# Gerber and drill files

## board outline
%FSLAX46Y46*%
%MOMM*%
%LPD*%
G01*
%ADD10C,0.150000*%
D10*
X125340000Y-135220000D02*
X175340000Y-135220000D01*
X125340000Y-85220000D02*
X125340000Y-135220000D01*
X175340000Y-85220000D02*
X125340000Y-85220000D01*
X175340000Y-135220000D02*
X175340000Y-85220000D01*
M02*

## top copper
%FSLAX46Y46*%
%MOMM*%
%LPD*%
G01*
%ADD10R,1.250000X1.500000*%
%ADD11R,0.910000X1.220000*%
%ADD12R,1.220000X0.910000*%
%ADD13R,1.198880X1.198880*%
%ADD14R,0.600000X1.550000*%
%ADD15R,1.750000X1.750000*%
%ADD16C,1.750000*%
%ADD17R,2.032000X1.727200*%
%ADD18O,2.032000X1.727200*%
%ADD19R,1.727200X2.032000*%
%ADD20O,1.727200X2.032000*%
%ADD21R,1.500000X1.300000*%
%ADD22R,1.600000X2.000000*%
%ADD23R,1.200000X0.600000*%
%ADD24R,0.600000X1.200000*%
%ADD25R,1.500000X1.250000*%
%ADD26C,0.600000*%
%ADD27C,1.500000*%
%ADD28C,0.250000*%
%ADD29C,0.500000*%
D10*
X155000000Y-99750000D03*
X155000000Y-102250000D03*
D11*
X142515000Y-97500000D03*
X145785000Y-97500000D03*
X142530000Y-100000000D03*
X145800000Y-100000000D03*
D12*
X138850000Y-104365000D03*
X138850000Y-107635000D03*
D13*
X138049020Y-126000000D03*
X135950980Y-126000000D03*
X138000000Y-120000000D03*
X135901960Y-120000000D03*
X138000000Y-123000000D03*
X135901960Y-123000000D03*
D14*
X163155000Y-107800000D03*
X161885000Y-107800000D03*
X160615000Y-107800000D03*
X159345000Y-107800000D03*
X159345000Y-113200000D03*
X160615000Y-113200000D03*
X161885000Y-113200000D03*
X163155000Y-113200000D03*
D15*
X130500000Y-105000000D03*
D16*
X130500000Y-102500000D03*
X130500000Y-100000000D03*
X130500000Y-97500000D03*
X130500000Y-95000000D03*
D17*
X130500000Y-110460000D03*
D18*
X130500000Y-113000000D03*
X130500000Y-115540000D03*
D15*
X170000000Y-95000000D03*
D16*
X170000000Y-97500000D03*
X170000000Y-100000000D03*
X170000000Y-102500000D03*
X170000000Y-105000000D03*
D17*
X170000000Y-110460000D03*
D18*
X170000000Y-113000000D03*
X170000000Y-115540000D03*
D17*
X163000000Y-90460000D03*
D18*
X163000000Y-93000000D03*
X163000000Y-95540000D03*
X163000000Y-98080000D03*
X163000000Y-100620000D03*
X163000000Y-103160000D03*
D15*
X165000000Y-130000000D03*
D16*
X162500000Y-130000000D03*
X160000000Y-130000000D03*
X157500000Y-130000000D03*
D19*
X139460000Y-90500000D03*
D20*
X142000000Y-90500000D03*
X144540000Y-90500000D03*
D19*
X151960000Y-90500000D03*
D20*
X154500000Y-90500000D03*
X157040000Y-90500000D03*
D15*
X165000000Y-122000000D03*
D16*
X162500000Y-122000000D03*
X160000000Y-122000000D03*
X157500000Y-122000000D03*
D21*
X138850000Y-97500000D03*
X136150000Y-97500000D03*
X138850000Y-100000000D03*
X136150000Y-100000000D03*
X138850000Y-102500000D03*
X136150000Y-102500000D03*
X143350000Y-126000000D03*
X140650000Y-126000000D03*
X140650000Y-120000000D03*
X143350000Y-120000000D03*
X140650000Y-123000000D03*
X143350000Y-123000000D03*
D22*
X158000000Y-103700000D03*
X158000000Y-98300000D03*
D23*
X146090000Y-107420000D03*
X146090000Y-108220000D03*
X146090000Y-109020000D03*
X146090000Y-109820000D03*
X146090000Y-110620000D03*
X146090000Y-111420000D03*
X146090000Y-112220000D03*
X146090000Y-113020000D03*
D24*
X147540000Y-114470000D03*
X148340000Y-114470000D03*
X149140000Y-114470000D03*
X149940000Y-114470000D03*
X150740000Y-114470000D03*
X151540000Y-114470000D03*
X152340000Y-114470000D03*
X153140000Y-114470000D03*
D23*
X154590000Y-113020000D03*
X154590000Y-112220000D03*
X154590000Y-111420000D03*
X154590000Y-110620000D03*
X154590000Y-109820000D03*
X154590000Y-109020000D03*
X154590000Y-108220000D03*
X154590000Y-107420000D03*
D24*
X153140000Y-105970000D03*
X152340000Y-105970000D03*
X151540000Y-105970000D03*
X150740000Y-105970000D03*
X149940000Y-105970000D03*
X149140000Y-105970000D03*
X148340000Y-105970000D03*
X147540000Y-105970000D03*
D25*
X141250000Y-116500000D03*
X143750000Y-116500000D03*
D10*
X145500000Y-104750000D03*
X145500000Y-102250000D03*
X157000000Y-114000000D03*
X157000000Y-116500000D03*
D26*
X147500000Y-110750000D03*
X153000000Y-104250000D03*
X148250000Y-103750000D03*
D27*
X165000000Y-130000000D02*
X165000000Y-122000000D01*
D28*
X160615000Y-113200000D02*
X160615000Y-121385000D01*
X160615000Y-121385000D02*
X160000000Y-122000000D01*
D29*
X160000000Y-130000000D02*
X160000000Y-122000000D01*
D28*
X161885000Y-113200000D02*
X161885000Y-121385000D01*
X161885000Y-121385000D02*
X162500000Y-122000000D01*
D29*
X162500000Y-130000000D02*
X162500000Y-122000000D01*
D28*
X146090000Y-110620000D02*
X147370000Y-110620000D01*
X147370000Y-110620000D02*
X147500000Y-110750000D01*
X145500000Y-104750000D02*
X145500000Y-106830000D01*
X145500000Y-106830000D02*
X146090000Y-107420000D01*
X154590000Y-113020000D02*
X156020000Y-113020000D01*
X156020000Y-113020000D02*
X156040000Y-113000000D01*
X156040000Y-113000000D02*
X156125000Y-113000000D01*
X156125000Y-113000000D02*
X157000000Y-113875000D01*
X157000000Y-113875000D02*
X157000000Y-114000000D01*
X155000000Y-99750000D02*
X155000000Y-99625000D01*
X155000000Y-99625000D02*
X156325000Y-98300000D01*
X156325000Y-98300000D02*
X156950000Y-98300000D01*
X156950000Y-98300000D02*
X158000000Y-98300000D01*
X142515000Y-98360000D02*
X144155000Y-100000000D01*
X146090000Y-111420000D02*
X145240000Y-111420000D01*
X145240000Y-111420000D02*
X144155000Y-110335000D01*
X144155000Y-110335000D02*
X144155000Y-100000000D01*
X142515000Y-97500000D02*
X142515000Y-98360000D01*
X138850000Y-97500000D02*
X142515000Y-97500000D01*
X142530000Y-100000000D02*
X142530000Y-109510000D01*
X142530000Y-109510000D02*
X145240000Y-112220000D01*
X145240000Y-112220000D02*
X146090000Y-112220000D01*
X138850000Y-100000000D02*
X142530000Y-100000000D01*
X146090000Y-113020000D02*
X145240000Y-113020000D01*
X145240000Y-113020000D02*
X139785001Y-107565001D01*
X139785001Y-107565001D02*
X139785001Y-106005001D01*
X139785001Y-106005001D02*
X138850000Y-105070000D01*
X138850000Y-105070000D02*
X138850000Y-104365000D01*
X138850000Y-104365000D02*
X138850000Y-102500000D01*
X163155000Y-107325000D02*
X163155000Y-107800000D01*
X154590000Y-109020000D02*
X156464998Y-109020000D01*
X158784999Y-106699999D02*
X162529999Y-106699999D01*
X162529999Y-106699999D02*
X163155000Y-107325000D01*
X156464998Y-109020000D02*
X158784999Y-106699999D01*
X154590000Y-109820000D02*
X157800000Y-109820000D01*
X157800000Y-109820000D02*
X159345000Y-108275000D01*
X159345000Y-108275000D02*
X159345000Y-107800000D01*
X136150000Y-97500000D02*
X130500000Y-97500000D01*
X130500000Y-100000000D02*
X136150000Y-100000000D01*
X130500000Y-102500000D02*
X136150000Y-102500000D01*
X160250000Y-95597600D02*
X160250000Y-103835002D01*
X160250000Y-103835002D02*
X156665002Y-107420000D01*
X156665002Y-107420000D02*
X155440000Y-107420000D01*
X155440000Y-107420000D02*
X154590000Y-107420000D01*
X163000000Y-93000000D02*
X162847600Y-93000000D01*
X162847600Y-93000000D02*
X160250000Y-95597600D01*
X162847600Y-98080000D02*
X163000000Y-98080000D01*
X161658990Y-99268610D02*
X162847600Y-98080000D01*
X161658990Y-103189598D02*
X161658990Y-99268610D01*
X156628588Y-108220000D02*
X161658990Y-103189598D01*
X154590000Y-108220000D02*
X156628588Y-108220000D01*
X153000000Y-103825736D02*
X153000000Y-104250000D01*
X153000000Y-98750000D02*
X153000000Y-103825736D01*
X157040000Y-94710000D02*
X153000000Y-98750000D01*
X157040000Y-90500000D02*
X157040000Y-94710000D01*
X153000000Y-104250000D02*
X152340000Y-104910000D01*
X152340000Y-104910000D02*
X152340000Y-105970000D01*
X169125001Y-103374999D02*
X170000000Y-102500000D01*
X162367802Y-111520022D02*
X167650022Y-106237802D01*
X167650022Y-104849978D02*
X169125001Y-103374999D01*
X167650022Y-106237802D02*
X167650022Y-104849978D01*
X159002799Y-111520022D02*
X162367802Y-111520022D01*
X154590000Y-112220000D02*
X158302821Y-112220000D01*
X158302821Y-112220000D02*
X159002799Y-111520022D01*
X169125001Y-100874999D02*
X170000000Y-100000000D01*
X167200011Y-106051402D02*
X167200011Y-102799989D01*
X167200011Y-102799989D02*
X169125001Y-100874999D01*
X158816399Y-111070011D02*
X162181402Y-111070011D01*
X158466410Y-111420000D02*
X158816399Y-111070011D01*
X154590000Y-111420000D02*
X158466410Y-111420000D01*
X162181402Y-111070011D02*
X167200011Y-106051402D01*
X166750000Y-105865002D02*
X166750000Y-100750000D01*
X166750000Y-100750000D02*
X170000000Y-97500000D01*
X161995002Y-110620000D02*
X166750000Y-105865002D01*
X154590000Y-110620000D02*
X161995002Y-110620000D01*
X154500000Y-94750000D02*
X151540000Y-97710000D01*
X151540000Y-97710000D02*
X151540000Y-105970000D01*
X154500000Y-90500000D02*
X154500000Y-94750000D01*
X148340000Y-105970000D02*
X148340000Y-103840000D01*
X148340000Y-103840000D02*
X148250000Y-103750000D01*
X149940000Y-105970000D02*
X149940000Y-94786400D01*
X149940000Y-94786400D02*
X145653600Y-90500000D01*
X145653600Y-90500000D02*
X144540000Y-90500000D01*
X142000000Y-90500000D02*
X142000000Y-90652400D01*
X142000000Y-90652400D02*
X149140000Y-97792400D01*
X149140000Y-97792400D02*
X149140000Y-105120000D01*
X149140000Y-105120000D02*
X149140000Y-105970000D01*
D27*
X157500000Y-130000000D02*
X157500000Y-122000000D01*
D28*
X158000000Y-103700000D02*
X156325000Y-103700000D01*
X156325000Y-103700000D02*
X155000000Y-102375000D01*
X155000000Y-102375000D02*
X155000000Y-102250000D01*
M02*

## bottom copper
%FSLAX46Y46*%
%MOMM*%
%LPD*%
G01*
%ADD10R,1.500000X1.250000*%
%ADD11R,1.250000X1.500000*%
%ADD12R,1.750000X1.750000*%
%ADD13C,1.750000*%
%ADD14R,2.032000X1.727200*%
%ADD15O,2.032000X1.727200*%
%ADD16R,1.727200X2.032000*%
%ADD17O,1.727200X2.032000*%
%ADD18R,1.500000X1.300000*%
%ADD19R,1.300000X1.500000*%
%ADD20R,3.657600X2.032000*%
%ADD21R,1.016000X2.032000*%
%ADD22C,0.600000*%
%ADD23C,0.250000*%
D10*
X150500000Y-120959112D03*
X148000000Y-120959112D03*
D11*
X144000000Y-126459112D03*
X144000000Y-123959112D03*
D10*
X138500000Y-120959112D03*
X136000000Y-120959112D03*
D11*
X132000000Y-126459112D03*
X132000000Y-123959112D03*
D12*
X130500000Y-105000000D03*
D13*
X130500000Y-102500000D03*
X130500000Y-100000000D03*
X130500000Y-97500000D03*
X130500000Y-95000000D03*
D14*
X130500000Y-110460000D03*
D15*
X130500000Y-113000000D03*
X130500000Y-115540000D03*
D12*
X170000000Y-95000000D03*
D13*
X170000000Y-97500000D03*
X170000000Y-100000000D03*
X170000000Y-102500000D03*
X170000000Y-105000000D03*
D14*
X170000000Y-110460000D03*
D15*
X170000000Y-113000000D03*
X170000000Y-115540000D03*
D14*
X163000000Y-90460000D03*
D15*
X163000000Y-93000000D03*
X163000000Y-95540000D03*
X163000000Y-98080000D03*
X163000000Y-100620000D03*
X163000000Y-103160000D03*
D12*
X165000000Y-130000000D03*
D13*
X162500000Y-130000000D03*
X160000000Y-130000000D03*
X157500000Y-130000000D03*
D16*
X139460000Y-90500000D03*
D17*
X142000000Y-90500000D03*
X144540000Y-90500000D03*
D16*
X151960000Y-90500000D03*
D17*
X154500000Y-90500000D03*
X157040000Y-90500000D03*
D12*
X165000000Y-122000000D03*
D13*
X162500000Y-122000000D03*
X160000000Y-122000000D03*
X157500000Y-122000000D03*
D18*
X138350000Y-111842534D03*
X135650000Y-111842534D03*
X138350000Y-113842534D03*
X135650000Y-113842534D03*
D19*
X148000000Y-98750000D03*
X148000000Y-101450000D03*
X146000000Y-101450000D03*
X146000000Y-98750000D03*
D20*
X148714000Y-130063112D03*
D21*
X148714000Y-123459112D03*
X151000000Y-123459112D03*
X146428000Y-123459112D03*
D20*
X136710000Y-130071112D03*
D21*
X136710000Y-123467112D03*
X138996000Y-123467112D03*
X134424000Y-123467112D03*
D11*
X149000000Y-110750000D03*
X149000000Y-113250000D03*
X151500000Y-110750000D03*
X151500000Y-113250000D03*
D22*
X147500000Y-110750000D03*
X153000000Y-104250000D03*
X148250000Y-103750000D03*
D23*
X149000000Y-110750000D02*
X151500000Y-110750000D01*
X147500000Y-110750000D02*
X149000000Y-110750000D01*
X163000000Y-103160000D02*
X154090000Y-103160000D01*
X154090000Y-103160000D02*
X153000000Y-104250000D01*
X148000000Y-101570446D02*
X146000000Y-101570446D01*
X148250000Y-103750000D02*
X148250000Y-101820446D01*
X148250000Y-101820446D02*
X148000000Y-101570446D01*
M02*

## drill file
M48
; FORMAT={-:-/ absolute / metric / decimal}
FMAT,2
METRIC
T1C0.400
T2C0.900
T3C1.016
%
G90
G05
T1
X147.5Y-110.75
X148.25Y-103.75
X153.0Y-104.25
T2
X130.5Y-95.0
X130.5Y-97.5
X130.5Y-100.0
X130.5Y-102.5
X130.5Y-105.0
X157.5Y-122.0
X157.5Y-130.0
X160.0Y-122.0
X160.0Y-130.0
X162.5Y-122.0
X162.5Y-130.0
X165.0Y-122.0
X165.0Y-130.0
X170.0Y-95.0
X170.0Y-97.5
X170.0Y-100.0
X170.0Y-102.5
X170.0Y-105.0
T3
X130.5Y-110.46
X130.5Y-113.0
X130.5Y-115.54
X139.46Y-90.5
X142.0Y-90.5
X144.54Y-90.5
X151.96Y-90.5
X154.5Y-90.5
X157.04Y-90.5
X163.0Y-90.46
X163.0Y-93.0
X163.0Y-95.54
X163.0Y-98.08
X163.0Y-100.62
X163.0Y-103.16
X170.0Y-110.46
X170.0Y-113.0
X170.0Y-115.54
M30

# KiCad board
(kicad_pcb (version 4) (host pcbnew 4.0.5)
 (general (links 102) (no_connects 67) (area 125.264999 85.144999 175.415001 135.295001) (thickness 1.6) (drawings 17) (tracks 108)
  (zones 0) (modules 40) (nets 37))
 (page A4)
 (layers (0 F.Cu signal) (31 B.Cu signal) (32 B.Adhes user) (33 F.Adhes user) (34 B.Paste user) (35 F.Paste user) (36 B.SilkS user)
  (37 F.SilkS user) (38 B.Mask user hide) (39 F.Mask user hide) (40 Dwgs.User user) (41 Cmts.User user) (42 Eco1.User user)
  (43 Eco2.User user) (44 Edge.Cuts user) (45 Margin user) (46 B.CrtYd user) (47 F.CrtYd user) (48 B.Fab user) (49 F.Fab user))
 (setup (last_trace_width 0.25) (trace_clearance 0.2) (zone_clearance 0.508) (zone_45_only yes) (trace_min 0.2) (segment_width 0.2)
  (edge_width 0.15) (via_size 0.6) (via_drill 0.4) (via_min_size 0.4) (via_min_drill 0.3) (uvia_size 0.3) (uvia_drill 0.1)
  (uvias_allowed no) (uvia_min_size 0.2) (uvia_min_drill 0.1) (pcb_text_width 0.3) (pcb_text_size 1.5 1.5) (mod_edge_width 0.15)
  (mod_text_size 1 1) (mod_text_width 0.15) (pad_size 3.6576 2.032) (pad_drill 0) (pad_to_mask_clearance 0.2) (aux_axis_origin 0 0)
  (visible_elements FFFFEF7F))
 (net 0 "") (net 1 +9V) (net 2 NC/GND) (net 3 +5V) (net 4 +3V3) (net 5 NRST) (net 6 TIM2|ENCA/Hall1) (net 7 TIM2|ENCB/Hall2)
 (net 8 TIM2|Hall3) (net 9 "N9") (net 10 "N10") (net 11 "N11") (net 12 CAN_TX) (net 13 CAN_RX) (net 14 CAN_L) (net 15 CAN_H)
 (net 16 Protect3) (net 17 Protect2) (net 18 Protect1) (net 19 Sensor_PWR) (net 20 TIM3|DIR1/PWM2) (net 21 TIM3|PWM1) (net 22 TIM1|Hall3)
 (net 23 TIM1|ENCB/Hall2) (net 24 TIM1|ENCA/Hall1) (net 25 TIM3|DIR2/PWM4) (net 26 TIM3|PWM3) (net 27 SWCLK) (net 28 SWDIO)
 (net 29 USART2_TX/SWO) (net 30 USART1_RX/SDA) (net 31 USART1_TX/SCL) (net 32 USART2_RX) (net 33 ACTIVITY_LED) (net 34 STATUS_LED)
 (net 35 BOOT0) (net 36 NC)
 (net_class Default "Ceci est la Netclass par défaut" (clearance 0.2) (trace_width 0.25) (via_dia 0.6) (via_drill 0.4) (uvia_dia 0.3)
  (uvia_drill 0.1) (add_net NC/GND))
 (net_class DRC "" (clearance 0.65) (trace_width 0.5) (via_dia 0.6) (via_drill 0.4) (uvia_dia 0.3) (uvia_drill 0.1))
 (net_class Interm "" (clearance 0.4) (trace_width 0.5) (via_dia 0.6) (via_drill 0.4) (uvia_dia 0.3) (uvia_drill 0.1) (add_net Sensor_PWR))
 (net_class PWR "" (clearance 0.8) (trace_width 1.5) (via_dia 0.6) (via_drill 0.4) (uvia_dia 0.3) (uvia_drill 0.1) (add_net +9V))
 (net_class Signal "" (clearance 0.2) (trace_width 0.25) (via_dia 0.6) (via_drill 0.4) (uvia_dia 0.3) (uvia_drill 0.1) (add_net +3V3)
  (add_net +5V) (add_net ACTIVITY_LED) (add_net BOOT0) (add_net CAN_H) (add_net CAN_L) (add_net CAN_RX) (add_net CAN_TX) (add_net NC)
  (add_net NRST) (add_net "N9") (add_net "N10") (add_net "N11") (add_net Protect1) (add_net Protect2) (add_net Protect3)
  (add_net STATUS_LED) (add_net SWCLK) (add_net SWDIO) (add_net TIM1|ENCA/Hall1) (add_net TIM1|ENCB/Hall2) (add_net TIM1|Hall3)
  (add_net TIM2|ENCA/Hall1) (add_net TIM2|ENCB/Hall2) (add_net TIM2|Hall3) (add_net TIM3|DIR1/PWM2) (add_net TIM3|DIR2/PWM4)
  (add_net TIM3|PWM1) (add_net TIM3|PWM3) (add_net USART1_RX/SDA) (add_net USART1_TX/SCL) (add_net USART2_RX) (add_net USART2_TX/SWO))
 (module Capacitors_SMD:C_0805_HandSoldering (layer B.Cu) (at 149.25 120.959112 180)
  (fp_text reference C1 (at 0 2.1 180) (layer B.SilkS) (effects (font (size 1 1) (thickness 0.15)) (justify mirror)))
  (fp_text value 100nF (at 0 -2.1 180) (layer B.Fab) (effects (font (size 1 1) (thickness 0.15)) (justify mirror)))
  (pad 1 smd rect (at -1.25 0 180) (size 1.5 1.25) (layers B.Cu B.Paste B.Mask) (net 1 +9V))
  (pad 2 smd rect (at 1.25 0 180) (size 1.5 1.25) (layers B.Cu B.Paste B.Mask) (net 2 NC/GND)))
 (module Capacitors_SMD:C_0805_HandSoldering (layer B.Cu) (at 144 125.209112 90)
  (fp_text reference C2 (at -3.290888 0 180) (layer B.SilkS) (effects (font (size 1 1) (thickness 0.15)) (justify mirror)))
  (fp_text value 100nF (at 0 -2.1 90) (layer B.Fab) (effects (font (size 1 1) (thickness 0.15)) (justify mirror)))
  (pad 1 smd rect (at -1.25 0 90) (size 1.5 1.25) (layers B.Cu B.Paste B.Mask) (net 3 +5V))
  (pad 2 smd rect (at 1.25 0 90) (size 1.5 1.25) (layers B.Cu B.Paste B.Mask) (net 2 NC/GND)))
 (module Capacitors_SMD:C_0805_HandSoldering (layer B.Cu) (at 137.25 120.959112 180)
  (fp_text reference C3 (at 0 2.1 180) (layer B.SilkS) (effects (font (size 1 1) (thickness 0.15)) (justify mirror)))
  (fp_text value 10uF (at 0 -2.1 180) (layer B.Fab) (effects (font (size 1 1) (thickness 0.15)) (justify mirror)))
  (pad 1 smd rect (at -1.25 0 180) (size 1.5 1.25) (layers B.Cu B.Paste B.Mask) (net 3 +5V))
  (pad 2 smd rect (at 1.25 0 180) (size 1.5 1.25) (layers B.Cu B.Paste B.Mask) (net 2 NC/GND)))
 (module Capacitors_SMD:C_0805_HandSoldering (layer B.Cu) (at 132 125.209112 90)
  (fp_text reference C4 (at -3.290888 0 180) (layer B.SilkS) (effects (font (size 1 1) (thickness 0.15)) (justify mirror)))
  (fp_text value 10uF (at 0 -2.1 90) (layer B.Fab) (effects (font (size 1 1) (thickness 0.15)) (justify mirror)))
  (pad 1 smd rect (at -1.25 0 90) (size 1.5 1.25) (layers B.Cu B.Paste B.Mask) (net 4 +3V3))
  (pad 2 smd rect (at 1.25 0 90) (size 1.5 1.25) (layers B.Cu B.Paste B.Mask) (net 2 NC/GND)))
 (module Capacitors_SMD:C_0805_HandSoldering (layer F.Cu) (at 155 101 270)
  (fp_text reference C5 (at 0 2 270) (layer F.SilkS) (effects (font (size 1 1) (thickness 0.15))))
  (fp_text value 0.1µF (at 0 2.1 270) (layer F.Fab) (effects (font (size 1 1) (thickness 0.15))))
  (pad 1 smd rect (at -1.25 0 270) (size 1.5 1.25) (layers F.Cu F.Paste F.Mask) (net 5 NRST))
  (pad 2 smd rect (at 1.25 0 270) (size 1.5 1.25) (layers F.Cu F.Paste F.Mask) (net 2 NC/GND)))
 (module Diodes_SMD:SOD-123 (layer F.Cu) (at 144.15 97.5)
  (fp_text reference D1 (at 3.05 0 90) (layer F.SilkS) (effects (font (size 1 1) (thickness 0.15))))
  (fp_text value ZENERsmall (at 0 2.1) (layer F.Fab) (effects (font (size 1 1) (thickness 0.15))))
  (pad 1 smd rect (at -1.635 0) (size 0.91 1.22) (layers F.Cu F.Paste F.Mask) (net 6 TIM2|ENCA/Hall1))
  (pad 2 smd rect (at 1.635 0) (size 0.91 1.22) (layers F.Cu F.Paste F.Mask) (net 2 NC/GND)))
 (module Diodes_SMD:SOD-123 (layer F.Cu) (at 144.165 100)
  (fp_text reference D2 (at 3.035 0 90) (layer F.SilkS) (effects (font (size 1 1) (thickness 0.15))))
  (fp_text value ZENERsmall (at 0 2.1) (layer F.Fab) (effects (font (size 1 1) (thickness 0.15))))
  (pad 1 smd rect (at -1.635 0) (size 0.91 1.22) (layers F.Cu F.Paste F.Mask) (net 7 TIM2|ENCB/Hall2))
  (pad 2 smd rect (at 1.635 0) (size 0.91 1.22) (layers F.Cu F.Paste F.Mask) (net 2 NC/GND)))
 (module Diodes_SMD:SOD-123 (layer F.Cu) (at 138.85 106 270)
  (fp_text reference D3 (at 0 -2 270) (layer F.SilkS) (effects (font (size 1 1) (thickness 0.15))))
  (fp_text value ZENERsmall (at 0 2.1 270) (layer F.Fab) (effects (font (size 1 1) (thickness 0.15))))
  (pad 1 smd rect (at -1.635 0 270) (size 0.91 1.22) (layers F.Cu F.Paste F.Mask) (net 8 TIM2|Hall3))
  (pad 2 smd rect (at 1.635 0 270) (size 0.91 1.22) (layers F.Cu F.Paste F.Mask) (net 2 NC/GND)))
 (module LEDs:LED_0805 (layer F.Cu) (at 137 126)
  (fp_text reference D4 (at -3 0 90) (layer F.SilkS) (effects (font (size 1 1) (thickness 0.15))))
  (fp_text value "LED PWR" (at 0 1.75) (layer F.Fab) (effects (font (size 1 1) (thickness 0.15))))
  (pad 2 smd rect (at 1.04902 0 180) (size 1.19888 1.19888) (layers F.Cu F.Paste F.Mask) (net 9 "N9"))
  (pad 1 smd rect (at -1.04902 0 180) (size 1.19888 1.19888) (layers F.Cu F.Paste F.Mask) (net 2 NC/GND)))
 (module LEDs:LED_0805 (layer F.Cu) (at 136.95098 120)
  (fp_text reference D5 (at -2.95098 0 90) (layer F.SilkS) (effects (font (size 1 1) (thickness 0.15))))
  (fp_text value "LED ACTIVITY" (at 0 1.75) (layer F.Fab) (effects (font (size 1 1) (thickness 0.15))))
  (pad 2 smd rect (at 1.04902 0 180) (size 1.19888 1.19888) (layers F.Cu F.Paste F.Mask) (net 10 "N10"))
  (pad 1 smd rect (at -1.04902 0 180) (size 1.19888 1.19888) (layers F.Cu F.Paste F.Mask) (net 2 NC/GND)))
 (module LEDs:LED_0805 (layer F.Cu) (at 136.95098 123)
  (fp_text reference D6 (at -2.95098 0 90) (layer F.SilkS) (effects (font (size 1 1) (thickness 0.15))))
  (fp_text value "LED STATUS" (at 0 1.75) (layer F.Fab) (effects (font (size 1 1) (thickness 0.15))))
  (pad 2 smd rect (at 1.04902 0 180) (size 1.19888 1.19888) (layers F.Cu F.Paste F.Mask) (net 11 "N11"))
  (pad 1 smd rect (at -1.04902 0 180) (size 1.19888 1.19888) (layers F.Cu F.Paste F.Mask) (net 2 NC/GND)))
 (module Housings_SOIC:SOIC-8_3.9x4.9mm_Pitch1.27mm (layer F.Cu) (at 161.25 110.5 270)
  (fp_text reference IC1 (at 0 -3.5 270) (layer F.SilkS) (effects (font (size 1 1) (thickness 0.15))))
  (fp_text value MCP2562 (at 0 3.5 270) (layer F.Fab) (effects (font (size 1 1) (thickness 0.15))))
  (pad 1 smd rect (at -2.7 -1.905 270) (size 1.55 0.6) (layers F.Cu F.Paste F.Mask) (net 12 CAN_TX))
  (pad 2 smd rect (at -2.7 -0.635 270) (size 1.55 0.6) (layers F.Cu F.Paste F.Mask) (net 2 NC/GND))
  (pad 3 smd rect (at -2.7 0.635 270) (size 1.55 0.6) (layers F.Cu F.Paste F.Mask) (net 3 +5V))
  (pad 4 smd rect (at -2.7 1.905 270) (size 1.55 0.6) (layers F.Cu F.Paste F.Mask) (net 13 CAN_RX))
  (pad 5 smd rect (at 2.7 1.905 270) (size 1.55 0.6) (layers F.Cu F.Paste F.Mask) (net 4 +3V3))
  (pad 6 smd rect (at 2.7 0.635 270) (size 1.55 0.6) (layers F.Cu F.Paste F.Mask) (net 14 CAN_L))
  (pad 7 smd rect (at 2.7 -0.635 270) (size 1.55 0.6) (layers F.Cu F.Paste F.Mask) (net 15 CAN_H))
  (pad 8 smd rect (at 2.7 -1.905 270) (size 1.55 0.6) (layers F.Cu F.Paste F.Mask) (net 2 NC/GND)))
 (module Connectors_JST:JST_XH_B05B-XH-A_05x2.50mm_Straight (layer F.Cu) (at 130.5 105 90)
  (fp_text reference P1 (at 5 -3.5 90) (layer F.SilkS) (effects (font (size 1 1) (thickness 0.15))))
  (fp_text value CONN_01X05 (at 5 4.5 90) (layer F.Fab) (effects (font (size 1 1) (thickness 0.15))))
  (pad 1 thru_hole rect (at 0 0 90) (size 1.75 1.75) (drill 0.9) (layers *.Cu *.Mask) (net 2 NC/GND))
  (pad 2 thru_hole circle (at 2.5 0 90) (size 1.75 1.75) (drill 0.9) (layers *.Cu *.Mask) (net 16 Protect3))
  (pad 3 thru_hole circle (at 5 0 90) (size 1.75 1.75) (drill 0.9) (layers *.Cu *.Mask) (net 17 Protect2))
  (pad 4 thru_hole circle (at 7.5 0 90) (size 1.75 1.75) (drill 0.9) (layers *.Cu *.Mask) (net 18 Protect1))
  (pad 5 thru_hole circle (at 10 0 90) (size 1.75 1.75) (drill 0.9) (layers *.Cu *.Mask) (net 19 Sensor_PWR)))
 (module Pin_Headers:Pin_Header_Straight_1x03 (layer F.Cu) (at 130.5 110.46)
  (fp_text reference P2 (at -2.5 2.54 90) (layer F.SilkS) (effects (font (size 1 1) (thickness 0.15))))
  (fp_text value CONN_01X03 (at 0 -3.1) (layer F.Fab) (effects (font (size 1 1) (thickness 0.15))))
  (pad 1 thru_hole rect (at 0 0) (size 2.032 1.7272) (drill 1.016) (layers *.Cu *.Mask F.SilkS) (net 2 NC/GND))
  (pad 2 thru_hole oval (at 0 2.54) (size 2.032 1.7272) (drill 1.016) (layers *.Cu *.Mask F.SilkS) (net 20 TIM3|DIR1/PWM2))
  (pad 3 thru_hole oval (at 0 5.08) (size 2.032 1.7272) (drill 1.016) (layers *.Cu *.Mask F.SilkS) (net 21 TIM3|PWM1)))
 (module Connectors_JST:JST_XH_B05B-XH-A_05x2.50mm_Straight (layer F.Cu) (at 170 95 270)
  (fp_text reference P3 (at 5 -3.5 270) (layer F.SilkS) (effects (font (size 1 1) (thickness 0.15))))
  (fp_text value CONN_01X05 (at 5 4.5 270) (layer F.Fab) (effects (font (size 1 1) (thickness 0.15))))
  (pad 1 thru_hole rect (at 0 0 270) (size 1.75 1.75) (drill 0.9) (layers *.Cu *.Mask) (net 2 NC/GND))
  (pad 2 thru_hole circle (at 2.5 0 270) (size 1.75 1.75) (drill 0.9) (layers *.Cu *.Mask) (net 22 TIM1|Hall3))
  (pad 3 thru_hole circle (at 5 0 270) (size 1.75 1.75) (drill 0.9) (layers *.Cu *.Mask) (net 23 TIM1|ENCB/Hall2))
  (pad 4 thru_hole circle (at 7.5 0 270) (size 1.75 1.75) (drill 0.9) (layers *.Cu *.Mask) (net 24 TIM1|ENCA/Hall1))
  (pad 5 thru_hole circle (at 10 0 270) (size 1.75 1.75) (drill 0.9) (layers *.Cu *.Mask) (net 19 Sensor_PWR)))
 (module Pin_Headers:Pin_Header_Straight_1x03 (layer F.Cu) (at 170 110.46)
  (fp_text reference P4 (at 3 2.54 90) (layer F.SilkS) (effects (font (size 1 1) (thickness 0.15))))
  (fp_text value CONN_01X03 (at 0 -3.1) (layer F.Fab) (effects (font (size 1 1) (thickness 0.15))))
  (pad 1 thru_hole rect (at 0 0) (size 2.032 1.7272) (drill 1.016) (layers *.Cu *.Mask F.SilkS) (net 2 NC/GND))
  (pad 2 thru_hole oval (at 0 2.54) (size 2.032 1.7272) (drill 1.016) (layers *.Cu *.Mask F.SilkS) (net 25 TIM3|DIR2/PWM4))
  (pad 3 thru_hole oval (at 0 5.08) (size 2.032 1.7272) (drill 1.016) (layers *.Cu *.Mask F.SilkS) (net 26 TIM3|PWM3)))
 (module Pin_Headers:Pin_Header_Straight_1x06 (layer F.Cu) (at 163 90.46)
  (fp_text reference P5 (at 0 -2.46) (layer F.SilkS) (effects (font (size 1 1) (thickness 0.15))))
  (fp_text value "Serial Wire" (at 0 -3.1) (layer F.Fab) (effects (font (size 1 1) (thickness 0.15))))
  (pad 1 thru_hole rect (at 0 0) (size 2.032 1.7272) (drill 1.016) (layers *.Cu *.Mask F.SilkS) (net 4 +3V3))
  (pad 2 thru_hole oval (at 0 2.54) (size 2.032 1.7272) (drill 1.016) (layers *.Cu *.Mask F.SilkS) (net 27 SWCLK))
  (pad 3 thru_hole oval (at 0 5.08) (size 2.032 1.7272) (drill 1.016) (layers *.Cu *.Mask F.SilkS) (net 2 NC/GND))
  (pad 4 thru_hole oval (at 0 7.62) (size 2.032 1.7272) (drill 1.016) (layers *.Cu *.Mask F.SilkS) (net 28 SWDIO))
  (pad 5 thru_hole oval (at 0 10.16) (size 2.032 1.7272) (drill 1.016) (layers *.Cu *.Mask F.SilkS) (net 5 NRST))
  (pad 6 thru_hole oval (at 0 12.7) (size 2.032 1.7272) (drill 1.016) (layers *.Cu *.Mask F.SilkS) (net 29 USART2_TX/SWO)))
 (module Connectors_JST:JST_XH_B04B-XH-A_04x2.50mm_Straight (layer F.Cu) (at 165 130 180)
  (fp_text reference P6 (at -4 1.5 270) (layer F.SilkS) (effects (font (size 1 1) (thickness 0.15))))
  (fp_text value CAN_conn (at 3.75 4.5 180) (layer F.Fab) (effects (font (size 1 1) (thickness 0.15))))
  (pad 1 thru_hole rect (at 0 0 180) (size 1.75 1.75) (drill 0.9) (layers *.Cu *.Mask) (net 1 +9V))
  (pad 2 thru_hole circle (at 2.5 0 180) (size 1.75 1.75) (drill 0.9) (layers *.Cu *.Mask) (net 15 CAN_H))
  (pad 3 thru_hole circle (at 5 0 180) (size 1.75 1.75) (drill 0.9) (layers *.Cu *.Mask) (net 14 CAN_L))
  (pad 4 thru_hole circle (at 7.5 0 180) (size 1.75 1.75) (drill 0.9) (layers *.Cu *.Mask) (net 2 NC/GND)))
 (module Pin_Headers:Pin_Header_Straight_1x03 (layer F.Cu) (at 139.46 90.5 90)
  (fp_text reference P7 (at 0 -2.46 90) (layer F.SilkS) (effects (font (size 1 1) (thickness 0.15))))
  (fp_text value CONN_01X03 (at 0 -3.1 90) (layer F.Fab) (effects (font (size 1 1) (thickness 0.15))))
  (pad 1 thru_hole rect (at 0 0 90) (size 2.032 1.7272) (drill 1.016) (layers *.Cu *.Mask F.SilkS) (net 2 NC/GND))
  (pad 2 thru_hole oval (at 0 2.54 90) (size 2.032 1.7272) (drill 1.016) (layers *.Cu *.Mask F.SilkS) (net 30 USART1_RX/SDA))
  (pad 3 thru_hole oval (at 0 5.08 90) (size 2.032 1.7272) (drill 1.016) (layers *.Cu *.Mask F.SilkS) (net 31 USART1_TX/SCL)))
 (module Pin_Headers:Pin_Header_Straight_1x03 (layer F.Cu) (at 151.96 90.5 90)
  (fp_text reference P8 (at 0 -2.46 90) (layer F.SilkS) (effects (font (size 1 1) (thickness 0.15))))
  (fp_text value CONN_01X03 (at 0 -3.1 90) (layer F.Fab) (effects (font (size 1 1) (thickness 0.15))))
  (pad 1 thru_hole rect (at 0 0 90) (size 2.032 1.7272) (drill 1.016) (layers *.Cu *.Mask F.SilkS) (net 2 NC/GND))
  (pad 2 thru_hole oval (at 0 2.54 90) (size 2.032 1.7272) (drill 1.016) (layers *.Cu *.Mask F.SilkS) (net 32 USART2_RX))
  (pad 3 thru_hole oval (at 0 5.08 90) (size 2.032 1.7272) (drill 1.016) (layers *.Cu *.Mask F.SilkS) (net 29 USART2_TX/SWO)))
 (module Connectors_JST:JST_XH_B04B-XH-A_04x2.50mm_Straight (layer F.Cu) (at 165 122 180)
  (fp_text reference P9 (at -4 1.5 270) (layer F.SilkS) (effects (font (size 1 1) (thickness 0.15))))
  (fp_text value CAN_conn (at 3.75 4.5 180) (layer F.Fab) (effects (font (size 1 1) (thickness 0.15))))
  (pad 1 thru_hole rect (at 0 0 180) (size 1.75 1.75) (drill 0.9) (layers *.Cu *.Mask) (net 1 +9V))
  (pad 2 thru_hole circle (at 2.5 0 180) (size 1.75 1.75) (drill 0.9) (layers *.Cu *.Mask) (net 15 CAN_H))
  (pad 3 thru_hole circle (at 5 0 180) (size 1.75 1.75) (drill 0.9) (layers *.Cu *.Mask) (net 14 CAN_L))
  (pad 4 thru_hole circle (at 7.5 0 180) (size 1.75 1.75) (drill 0.9) (layers *.Cu *.Mask) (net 2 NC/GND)))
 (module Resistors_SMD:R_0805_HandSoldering (layer F.Cu) (at 137.5 97.5 180)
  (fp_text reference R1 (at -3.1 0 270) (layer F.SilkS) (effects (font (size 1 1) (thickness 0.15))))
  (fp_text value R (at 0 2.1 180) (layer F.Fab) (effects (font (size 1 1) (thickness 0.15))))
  (pad 1 smd rect (at -1.35 0 180) (size 1.5 1.3) (layers F.Cu F.Paste F.Mask) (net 6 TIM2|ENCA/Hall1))
  (pad 2 smd rect (at 1.35 0 180) (size 1.5 1.3) (layers F.Cu F.Paste F.Mask) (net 18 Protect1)))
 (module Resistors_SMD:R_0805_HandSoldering (layer F.Cu) (at 137.5 100 180)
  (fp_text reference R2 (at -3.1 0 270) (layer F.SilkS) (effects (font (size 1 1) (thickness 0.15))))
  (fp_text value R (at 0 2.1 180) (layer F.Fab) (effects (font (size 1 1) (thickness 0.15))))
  (pad 1 smd rect (at -1.35 0 180) (size 1.5 1.3) (layers F.Cu F.Paste F.Mask) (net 7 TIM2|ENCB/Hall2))
  (pad 2 smd rect (at 1.35 0 180) (size 1.5 1.3) (layers F.Cu F.Paste F.Mask) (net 17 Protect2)))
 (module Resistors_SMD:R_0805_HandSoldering (layer F.Cu) (at 137.5 102.5 180)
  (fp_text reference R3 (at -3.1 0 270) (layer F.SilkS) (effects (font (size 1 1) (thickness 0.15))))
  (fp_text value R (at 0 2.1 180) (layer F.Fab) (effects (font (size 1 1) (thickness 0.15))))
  (pad 1 smd rect (at -1.35 0 180) (size 1.5 1.3) (layers F.Cu F.Paste F.Mask) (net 8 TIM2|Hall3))
  (pad 2 smd rect (at 1.35 0 180) (size 1.5 1.3) (layers F.Cu F.Paste F.Mask) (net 16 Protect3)))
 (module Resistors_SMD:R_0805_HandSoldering (layer F.Cu) (at 142 126 180)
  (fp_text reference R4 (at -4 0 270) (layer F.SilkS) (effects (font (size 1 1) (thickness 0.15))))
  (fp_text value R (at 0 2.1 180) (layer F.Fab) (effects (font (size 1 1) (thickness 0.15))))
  (pad 1 smd rect (at -1.35 0 180) (size 1.5 1.3) (layers F.Cu F.Paste F.Mask) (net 4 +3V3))
  (pad 2 smd rect (at 1.35 0 180) (size 1.5 1.3) (layers F.Cu F.Paste F.Mask) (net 9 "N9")))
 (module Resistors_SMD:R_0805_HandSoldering (layer B.Cu) (at 137 111.842534 180)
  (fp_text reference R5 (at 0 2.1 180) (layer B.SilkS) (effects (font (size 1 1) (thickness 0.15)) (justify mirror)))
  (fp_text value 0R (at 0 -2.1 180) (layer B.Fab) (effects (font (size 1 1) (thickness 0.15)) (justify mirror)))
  (pad 1 smd rect (at -1.35 0 180) (size 1.5 1.3) (layers B.Cu B.Paste B.Mask) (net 4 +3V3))
  (pad 2 smd rect (at 1.35 0 180) (size 1.5 1.3) (layers B.Cu B.Paste B.Mask) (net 19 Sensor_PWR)))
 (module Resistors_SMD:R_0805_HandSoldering (layer B.Cu) (at 137 113.842534 180)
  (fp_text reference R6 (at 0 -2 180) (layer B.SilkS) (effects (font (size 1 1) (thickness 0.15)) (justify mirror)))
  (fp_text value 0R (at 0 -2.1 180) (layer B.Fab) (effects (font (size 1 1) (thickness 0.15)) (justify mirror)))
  (pad 1 smd rect (at -1.35 0 180) (size 1.5 1.3) (layers B.Cu B.Paste B.Mask) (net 3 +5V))
  (pad 2 smd rect (at 1.35 0 180) (size 1.5 1.3) (layers B.Cu B.Paste B.Mask) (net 19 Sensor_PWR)))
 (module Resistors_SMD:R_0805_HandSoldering (layer F.Cu) (at 142 120)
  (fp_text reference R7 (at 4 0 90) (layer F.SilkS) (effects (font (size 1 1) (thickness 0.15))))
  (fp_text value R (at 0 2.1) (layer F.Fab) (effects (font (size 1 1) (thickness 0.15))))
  (pad 1 smd rect (at -1.35 0) (size 1.5 1.3) (layers F.Cu F.Paste F.Mask) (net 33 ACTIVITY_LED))
  (pad 2 smd rect (at 1.35 0) (size 1.5 1.3) (layers F.Cu F.Paste F.Mask) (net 10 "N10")))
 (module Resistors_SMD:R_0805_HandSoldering (layer F.Cu) (at 142 123)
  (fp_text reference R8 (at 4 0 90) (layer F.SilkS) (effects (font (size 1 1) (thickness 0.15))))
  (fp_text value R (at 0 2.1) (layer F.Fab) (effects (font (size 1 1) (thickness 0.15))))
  (pad 1 smd rect (at -1.35 0) (size 1.5 1.3) (layers F.Cu F.Paste F.Mask) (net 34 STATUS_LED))
  (pad 2 smd rect (at 1.35 0) (size 1.5 1.3) (layers F.Cu F.Paste F.Mask) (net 11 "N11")))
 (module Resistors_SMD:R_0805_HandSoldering (layer B.Cu) (at 148 100.1 270)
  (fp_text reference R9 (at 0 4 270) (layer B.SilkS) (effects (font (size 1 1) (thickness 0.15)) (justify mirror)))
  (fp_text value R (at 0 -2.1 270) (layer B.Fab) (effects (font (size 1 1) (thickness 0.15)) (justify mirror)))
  (pad 1 smd rect (at -1.35 0 270) (size 1.5 1.3) (layers B.Cu B.Paste B.Mask) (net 4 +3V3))
  (pad 2 smd rect (at 1.35 0 270) (size 1.5 1.3) (layers B.Cu B.Paste B.Mask) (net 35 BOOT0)))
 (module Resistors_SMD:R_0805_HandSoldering (layer B.Cu) (at 146 100.1 90)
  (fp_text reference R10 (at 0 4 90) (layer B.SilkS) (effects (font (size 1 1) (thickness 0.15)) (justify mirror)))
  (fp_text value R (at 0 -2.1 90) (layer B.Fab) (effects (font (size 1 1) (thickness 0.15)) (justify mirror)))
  (pad 1 smd rect (at -1.35 0 90) (size 1.5 1.3) (layers B.Cu B.Paste B.Mask) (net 35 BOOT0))
  (pad 2 smd rect (at 1.35 0 90) (size 1.5 1.3) (layers B.Cu B.Paste B.Mask) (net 2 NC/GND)))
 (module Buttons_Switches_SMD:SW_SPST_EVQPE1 (layer F.Cu) (at 158 101 270)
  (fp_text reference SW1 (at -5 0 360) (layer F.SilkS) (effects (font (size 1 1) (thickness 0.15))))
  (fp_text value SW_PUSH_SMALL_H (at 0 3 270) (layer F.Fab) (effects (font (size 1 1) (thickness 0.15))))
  (pad 2 smd rect (at 2.7 0 270) (size 2 1.6) (layers F.Cu F.Paste F.Mask) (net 2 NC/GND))
  (pad 1 smd rect (at -2.7 0 270) (size 2 1.6) (layers F.Cu F.Paste F.Mask) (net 5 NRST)))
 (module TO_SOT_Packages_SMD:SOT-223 (layer B.Cu) (at 148.714 126.761112)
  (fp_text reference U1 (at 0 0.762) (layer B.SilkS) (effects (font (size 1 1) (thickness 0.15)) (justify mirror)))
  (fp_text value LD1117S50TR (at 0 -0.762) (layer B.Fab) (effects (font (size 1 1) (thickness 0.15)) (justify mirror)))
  (pad 2 smd rect (at 0 3.302) (size 3.6576 2.032) (layers B.Cu B.Paste B.Mask) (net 3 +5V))
  (pad 2 smd rect (at 0 -3.302) (size 1.016 2.032) (layers B.Cu B.Paste B.Mask) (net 3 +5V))
  (pad 3 smd rect (at 2.286 -3.302) (size 1.016 2.032) (layers B.Cu B.Paste B.Mask) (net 1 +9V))
  (pad 1 smd rect (at -2.286 -3.302) (size 1.016 2.032) (layers B.Cu B.Paste B.Mask) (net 2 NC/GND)))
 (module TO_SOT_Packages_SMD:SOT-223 (layer B.Cu) (at 136.71 126.769112)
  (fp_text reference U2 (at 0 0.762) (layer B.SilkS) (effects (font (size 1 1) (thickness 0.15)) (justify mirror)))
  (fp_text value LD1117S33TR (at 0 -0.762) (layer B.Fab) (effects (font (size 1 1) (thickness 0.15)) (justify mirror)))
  (pad 2 smd rect (at 0 3.302) (size 3.6576 2.032) (layers B.Cu B.Paste B.Mask) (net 4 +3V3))
  (pad 2 smd rect (at 0 -3.302) (size 1.016 2.032) (layers B.Cu B.Paste B.Mask) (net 4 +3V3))
  (pad 3 smd rect (at 2.286 -3.302) (size 1.016 2.032) (layers B.Cu B.Paste B.Mask) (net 3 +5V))
  (pad 1 smd rect (at -2.286 -3.302) (size 1.016 2.032) (layers B.Cu B.Paste B.Mask) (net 2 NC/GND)))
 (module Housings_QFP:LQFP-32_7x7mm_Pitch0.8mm (layer F.Cu) (at 150.34 110.22)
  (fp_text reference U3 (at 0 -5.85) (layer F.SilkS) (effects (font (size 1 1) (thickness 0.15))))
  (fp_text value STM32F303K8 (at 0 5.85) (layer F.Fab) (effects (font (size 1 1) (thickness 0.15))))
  (pad 1 smd rect (at -4.25 -2.8) (size 1.2 0.6) (layers F.Cu F.Paste F.Mask) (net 4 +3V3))
  (pad 2 smd rect (at -4.25 -2) (size 1.2 0.6) (layers F.Cu F.Paste F.Mask) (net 34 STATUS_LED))
  (pad 3 smd rect (at -4.25 -1.2) (size 1.2 0.6) (layers F.Cu F.Paste F.Mask) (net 33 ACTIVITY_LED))
  (pad 4 smd rect (at -4.25 -0.4) (size 1.2 0.6) (layers F.Cu F.Paste F.Mask) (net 5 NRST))
  (pad 5 smd rect (at -4.25 0.4) (size 1.2 0.6) (layers F.Cu F.Paste F.Mask) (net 4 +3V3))
  (pad 6 smd rect (at -4.25 1.2) (size 1.2 0.6) (layers F.Cu F.Paste F.Mask) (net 6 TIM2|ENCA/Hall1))
  (pad 7 smd rect (at -4.25 2) (size 1.2 0.6) (layers F.Cu F.Paste F.Mask) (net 7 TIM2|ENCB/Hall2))
  (pad 8 smd rect (at -4.25 2.8) (size 1.2 0.6) (layers F.Cu F.Paste F.Mask) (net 8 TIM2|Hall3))
  (pad 9 smd rect (at -2.8 4.25 90) (size 1.2 0.6) (layers F.Cu F.Paste F.Mask) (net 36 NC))
  (pad 10 smd rect (at -2 4.25 90) (size 1.2 0.6) (layers F.Cu F.Paste F.Mask) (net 36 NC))
  (pad 11 smd rect (at -1.2 4.25 90) (size 1.2 0.6) (layers F.Cu F.Paste F.Mask) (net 36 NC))
  (pad 12 smd rect (at -0.4 4.25 90) (size 1.2 0.6) (layers F.Cu F.Paste F.Mask) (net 21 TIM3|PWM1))
  (pad 13 smd rect (at 0.4 4.25 90) (size 1.2 0.6) (layers F.Cu F.Paste F.Mask) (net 20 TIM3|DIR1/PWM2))
  (pad 14 smd rect (at 1.2 4.25 90) (size 1.2 0.6) (layers F.Cu F.Paste F.Mask) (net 26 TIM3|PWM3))
  (pad 15 smd rect (at 2 4.25 90) (size 1.2 0.6) (layers F.Cu F.Paste F.Mask) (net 25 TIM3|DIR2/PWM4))
  (pad 16 smd rect (at 2.8 4.25 90) (size 1.2 0.6) (layers F.Cu F.Paste F.Mask) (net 2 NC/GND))
  (pad 17 smd rect (at 4.25 2.8) (size 1.2 0.6) (layers F.Cu F.Paste F.Mask) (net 4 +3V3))
  (pad 18 smd rect (at 4.25 2) (size 1.2 0.6) (layers F.Cu F.Paste F.Mask) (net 24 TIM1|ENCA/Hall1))
  (pad 19 smd rect (at 4.25 1.2) (size 1.2 0.6) (layers F.Cu F.Paste F.Mask) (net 23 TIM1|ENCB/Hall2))
  (pad 20 smd rect (at 4.25 0.4) (size 1.2 0.6) (layers F.Cu F.Paste F.Mask) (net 22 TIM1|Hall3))
  (pad 21 smd rect (at 4.25 -0.4) (size 1.2 0.6) (layers F.Cu F.Paste F.Mask) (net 13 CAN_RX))
  (pad 22 smd rect (at 4.25 -1.2) (size 1.2 0.6) (layers F.Cu F.Paste F.Mask) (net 12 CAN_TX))
  (pad 23 smd rect (at 4.25 -2) (size 1.2 0.6) (layers F.Cu F.Paste F.Mask) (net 28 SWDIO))
  (pad 24 smd rect (at 4.25 -2.8) (size 1.2 0.6) (layers F.Cu F.Paste F.Mask) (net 27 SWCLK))
  (pad 25 smd rect (at 2.8 -4.25 90) (size 1.2 0.6) (layers F.Cu F.Paste F.Mask) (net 36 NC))
  (pad 26 smd rect (at 2 -4.25 90) (size 1.2 0.6) (layers F.Cu F.Paste F.Mask) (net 29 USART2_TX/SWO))
  (pad 27 smd rect (at 1.2 -4.25 90) (size 1.2 0.6) (layers F.Cu F.Paste F.Mask) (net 32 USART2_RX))
  (pad 28 smd rect (at 0.4 -4.25 90) (size 1.2 0.6) (layers F.Cu F.Paste F.Mask) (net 36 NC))
  (pad 29 smd rect (at -0.4 -4.25 90) (size 1.2 0.6) (layers F.Cu F.Paste F.Mask) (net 31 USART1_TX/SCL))
  (pad 30 smd rect (at -1.2 -4.25 90) (size 1.2 0.6) (layers F.Cu F.Paste F.Mask) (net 30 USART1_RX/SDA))
  (pad 31 smd rect (at -2 -4.25 90) (size 1.2 0.6) (layers F.Cu F.Paste F.Mask) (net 35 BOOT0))
  (pad 32 smd rect (at -2.8 -4.25 90) (size 1.2 0.6) (layers F.Cu F.Paste F.Mask) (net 2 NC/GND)))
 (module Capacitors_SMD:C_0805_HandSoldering (layer B.Cu) (at 149 112 270)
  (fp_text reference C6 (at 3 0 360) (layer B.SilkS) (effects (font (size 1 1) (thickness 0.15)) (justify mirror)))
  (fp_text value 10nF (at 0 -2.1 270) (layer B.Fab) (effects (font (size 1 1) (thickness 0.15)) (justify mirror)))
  (pad 1 smd rect (at -1.25 0 270) (size 1.5 1.25) (layers B.Cu B.Paste B.Mask) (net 4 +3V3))
  (pad 2 smd rect (at 1.25 0 270) (size 1.5 1.25) (layers B.Cu B.Paste B.Mask) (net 2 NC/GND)))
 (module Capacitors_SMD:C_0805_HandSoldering (layer B.Cu) (at 151.5 112 270)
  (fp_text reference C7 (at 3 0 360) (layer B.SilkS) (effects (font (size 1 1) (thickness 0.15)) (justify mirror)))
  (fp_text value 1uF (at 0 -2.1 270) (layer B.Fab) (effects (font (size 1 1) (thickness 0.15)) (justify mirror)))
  (pad 1 smd rect (at -1.25 0 270) (size 1.5 1.25) (layers B.Cu B.Paste B.Mask) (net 4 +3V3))
  (pad 2 smd rect (at 1.25 0 270) (size 1.5 1.25) (layers B.Cu B.Paste B.Mask) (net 2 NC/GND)))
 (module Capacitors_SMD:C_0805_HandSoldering (layer F.Cu) (at 142.5 116.5)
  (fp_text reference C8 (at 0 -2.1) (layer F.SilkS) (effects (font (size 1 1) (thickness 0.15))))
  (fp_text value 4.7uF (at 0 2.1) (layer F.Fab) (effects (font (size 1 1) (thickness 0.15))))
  (pad 1 smd rect (at -1.25 0) (size 1.5 1.25) (layers F.Cu F.Paste F.Mask) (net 4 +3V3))
  (pad 2 smd rect (at 1.25 0) (size 1.5 1.25) (layers F.Cu F.Paste F.Mask) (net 2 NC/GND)))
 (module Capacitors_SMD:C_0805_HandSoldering (layer F.Cu) (at 145.5 103.5 90)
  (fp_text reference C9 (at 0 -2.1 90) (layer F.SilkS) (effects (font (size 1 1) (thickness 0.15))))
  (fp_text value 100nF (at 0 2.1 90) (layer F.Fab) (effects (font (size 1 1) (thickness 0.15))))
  (pad 1 smd rect (at -1.25 0 90) (size 1.5 1.25) (layers F.Cu F.Paste F.Mask) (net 4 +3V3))
  (pad 2 smd rect (at 1.25 0 90) (size 1.5 1.25) (layers F.Cu F.Paste F.Mask) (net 2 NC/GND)))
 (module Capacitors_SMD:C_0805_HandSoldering (layer F.Cu) (at 157 115.25 270)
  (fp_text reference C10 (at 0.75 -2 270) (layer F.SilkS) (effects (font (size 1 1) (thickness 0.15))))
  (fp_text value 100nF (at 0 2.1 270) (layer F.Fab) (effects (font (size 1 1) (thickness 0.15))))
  (pad 1 smd rect (at -1.25 0 270) (size 1.5 1.25) (layers F.Cu F.Paste F.Mask) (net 4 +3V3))
  (pad 2 smd rect (at 1.25 0 270) (size 1.5 1.25) (layers F.Cu F.Paste F.Mask) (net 2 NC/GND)))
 (gr_line (start 125.34 135.22) (end 175.34 135.22) (layer Edge.Cuts) (width 0.15))
 (gr_line (start 125.34 85.22) (end 125.34 135.22) (layer Edge.Cuts) (width 0.15))
 (gr_line (start 175.34 85.22) (end 125.34 85.22) (layer Edge.Cuts) (width 0.15))
 (gr_line (start 175.34 135.22) (end 175.34 85.22) (layer Edge.Cuts) (width 0.15))
 (segment (start 165 130) (end 165 122) (width 1.5) (layer F.Cu) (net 1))
 (segment (start 160.615 113.2) (end 160.615 121.385) (width 0.25) (layer F.Cu) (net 14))
 (segment (start 160.615 121.385) (end 160 122) (width 0.25) (layer F.Cu) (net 14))
 (segment (start 160 130) (end 160 122) (width 0.5) (layer F.Cu) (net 14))
 (segment (start 161.885 113.2) (end 161.885 121.385) (width 0.25) (layer F.Cu) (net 15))
 (segment (start 161.885 121.385) (end 162.5 122) (width 0.25) (layer F.Cu) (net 15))
 (segment (start 162.5 130) (end 162.5 122) (width 0.5) (layer F.Cu) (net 15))
 (segment (start 149 110.75) (end 151.5 110.75) (width 0.25) (layer B.Cu) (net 4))
 (segment (start 147.5 110.75) (end 149 110.75) (width 0.25) (layer B.Cu) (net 4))
 (segment (start 146.09 110.62) (end 147.37 110.62) (width 0.25) (layer F.Cu) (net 4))
 (segment (start 147.37 110.62) (end 147.5 110.75) (width 0.25) (layer F.Cu) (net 4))
 (via (at 147.5 110.75) (size 0.6) (drill 0.4) (layers F.Cu B.Cu) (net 4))
 (segment (start 145.5 104.75) (end 145.5 106.83) (width 0.25) (layer F.Cu) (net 4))
 (segment (start 145.5 106.83) (end 146.09 107.42) (width 0.25) (layer F.Cu) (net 4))
 (segment (start 154.59 113.02) (end 156.02 113.02) (width 0.25) (layer F.Cu) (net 4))
 (segment (start 156.02 113.02) (end 156.04 113) (width 0.25) (layer F.Cu) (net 4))
 (segment (start 156.04 113) (end 156.125 113) (width 0.25) (layer F.Cu) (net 4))
 (segment (start 156.125 113) (end 157 113.875) (width 0.25) (layer F.Cu) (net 4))
 (segment (start 157 113.875) (end 157 114) (width 0.25) (layer F.Cu) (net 4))
 (segment (start 155 99.75) (end 155 99.625) (width 0.25) (layer F.Cu) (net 5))
 (segment (start 155 99.625) (end 156.325 98.3) (width 0.25) (layer F.Cu) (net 5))
 (segment (start 156.325 98.3) (end 156.95 98.3) (width 0.25) (layer F.Cu) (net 5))
 (segment (start 156.95 98.3) (end 158 98.3) (width 0.25) (layer F.Cu) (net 5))
 (segment (start 142.515 98.36) (end 144.155 100) (width 0.25) (layer F.Cu) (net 6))
 (segment (start 146.09 111.42) (end 145.24 111.42) (width 0.25) (layer F.Cu) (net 6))
 (segment (start 145.24 111.42) (end 144.155 110.335) (width 0.25) (layer F.Cu) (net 6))
 (segment (start 144.155 110.335) (end 144.155 100) (width 0.25) (layer F.Cu) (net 6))
 (segment (start 142.515 97.5) (end 142.515 98.36) (width 0.25) (layer F.Cu) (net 6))
 (segment (start 138.85 97.5) (end 142.515 97.5) (width 0.25) (layer F.Cu) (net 6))
 (segment (start 142.53 100) (end 142.53 109.51) (width 0.25) (layer F.Cu) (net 7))
 (segment (start 142.53 109.51) (end 145.24 112.22) (width 0.25) (layer F.Cu) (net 7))
 (segment (start 145.24 112.22) (end 146.09 112.22) (width 0.25) (layer F.Cu) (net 7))
 (segment (start 138.85 100) (end 142.53 100) (width 0.25) (layer F.Cu) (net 7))
 (segment (start 146.09 113.02) (end 145.24 113.02) (width 0.25) (layer F.Cu) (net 8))
 (segment (start 145.24 113.02) (end 139.785001 107.565001) (width 0.25) (layer F.Cu) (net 8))
 (segment (start 139.785001 107.565001) (end 139.785001 106.005001) (width 0.25) (layer F.Cu) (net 8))
 (segment (start 139.785001 106.005001) (end 138.85 105.07) (width 0.25) (layer F.Cu) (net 8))
 (segment (start 138.85 105.07) (end 138.85 104.365) (width 0.25) (layer F.Cu) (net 8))
 (segment (start 138.85 104.365) (end 138.85 102.5) (width 0.25) (layer F.Cu) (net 8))
 (segment (start 163.155 107.325) (end 163.155 107.8) (width 0.25) (layer F.Cu) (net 12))
 (segment (start 154.59 109.02) (end 156.464998 109.02) (width 0.25) (layer F.Cu) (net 12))
 (segment (start 158.784999 106.699999) (end 162.529999 106.699999) (width 0.25) (layer F.Cu) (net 12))
 (segment (start 162.529999 106.699999) (end 163.155 107.325) (width 0.25) (layer F.Cu) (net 12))
 (segment (start 156.464998 109.02) (end 158.784999 106.699999) (width 0.25) (layer F.Cu) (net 12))
 (segment (start 154.59 109.82) (end 157.8 109.82) (width 0.25) (layer F.Cu) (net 13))
 (segment (start 157.8 109.82) (end 159.345 108.275) (width 0.25) (layer F.Cu) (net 13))
 (segment (start 159.345 108.275) (end 159.345 107.8) (width 0.25) (layer F.Cu) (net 13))
 (segment (start 136.15 97.5) (end 130.5 97.5) (width 0.25) (layer F.Cu) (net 18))
 (segment (start 130.5 100) (end 136.15 100) (width 0.25) (layer F.Cu) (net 17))
 (segment (start 130.5 102.5) (end 136.15 102.5) (width 0.25) (layer F.Cu) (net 16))
 (segment (start 160.25 95.5976) (end 160.25 103.835002) (width 0.25) (layer F.Cu) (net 27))
 (segment (start 160.25 103.835002) (end 156.665002 107.42) (width 0.25) (layer F.Cu) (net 27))
 (segment (start 156.665002 107.42) (end 155.44 107.42) (width 0.25) (layer F.Cu) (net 27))
 (segment (start 155.44 107.42) (end 154.59 107.42) (width 0.25) (layer F.Cu) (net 27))
 (segment (start 163 93) (end 162.8476 93) (width 0.25) (layer F.Cu) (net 27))
 (segment (start 162.8476 93) (end 160.25 95.5976) (width 0.25) (layer F.Cu) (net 27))
 (segment (start 162.8476 98.08) (end 163 98.08) (width 0.25) (layer F.Cu) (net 28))
 (segment (start 161.65899 99.26861) (end 162.8476 98.08) (width 0.25) (layer F.Cu) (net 28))
 (segment (start 161.65899 103.189598) (end 161.65899 99.26861) (width 0.25) (layer F.Cu) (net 28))
 (segment (start 156.628588 108.22) (end 161.65899 103.189598) (width 0.25) (layer F.Cu) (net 28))
 (segment (start 154.59 108.22) (end 156.628588 108.22) (width 0.25) (layer F.Cu) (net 28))
 (segment (start 153 103.825736) (end 153 104.25) (width 0.25) (layer F.Cu) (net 29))
 (segment (start 153 98.75) (end 153 103.825736) (width 0.25) (layer F.Cu) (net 29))
 (segment (start 157.04 94.71) (end 153 98.75) (width 0.25) (layer F.Cu) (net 29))
 (segment (start 157.04 90.5) (end 157.04 94.71) (width 0.25) (layer F.Cu) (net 29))
 (segment (start 163 103.16) (end 154.09 103.16) (width 0.25) (layer B.Cu) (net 29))
 (segment (start 154.09 103.16) (end 153 104.25) (width 0.25) (layer B.Cu) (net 29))
 (segment (start 153 104.25) (end 152.34 104.91) (width 0.25) (layer F.Cu) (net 29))
 (segment (start 152.34 104.91) (end 152.34 105.97) (width 0.25) (layer F.Cu) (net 29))
 (via (at 153 104.25) (size 0.6) (drill 0.4) (layers F.Cu B.Cu) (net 29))
 (segment (start 169.125001 103.374999) (end 170 102.5) (width 0.25) (layer F.Cu) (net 24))
 (segment (start 162.367802 111.520022) (end 167.650022 106.237802) (width 0.25) (layer F.Cu) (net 24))
 (segment (start 167.650022 104.849978) (end 169.125001 103.374999) (width 0.25) (layer F.Cu) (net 24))
 (segment (start 167.650022 106.237802) (end 167.650022 104.849978) (width 0.25) (layer F.Cu) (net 24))
 (segment (start 159.002799 111.520022) (end 162.367802 111.520022) (width 0.25) (layer F.Cu) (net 24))
 (segment (start 154.59 112.22) (end 158.302821 112.22) (width 0.25) (layer F.Cu) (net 24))
 (segment (start 158.302821 112.22) (end 159.002799 111.520022) (width 0.25) (layer F.Cu) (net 24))
 (segment (start 169.125001 100.874999) (end 170 100) (width 0.25) (layer F.Cu) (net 23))
 (segment (start 167.200011 106.051402) (end 167.200011 102.799989) (width 0.25) (layer F.Cu) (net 23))
 (segment (start 167.200011 102.799989) (end 169.125001 100.874999) (width 0.25) (layer F.Cu) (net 23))
 (segment (start 158.816399 111.070011) (end 162.181402 111.070011) (width 0.25) (layer F.Cu) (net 23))
 (segment (start 158.46641 111.42) (end 158.816399 111.070011) (width 0.25) (layer F.Cu) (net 23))
 (segment (start 154.59 111.42) (end 158.46641 111.42) (width 0.25) (layer F.Cu) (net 23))
 (segment (start 162.181402 111.070011) (end 167.200011 106.051402) (width 0.25) (layer F.Cu) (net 23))
 (segment (start 166.75 105.865002) (end 166.75 100.75) (width 0.25) (layer F.Cu) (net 22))
 (segment (start 166.75 100.75) (end 170 97.5) (width 0.25) (layer F.Cu) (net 22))
 (segment (start 161.995002 110.62) (end 166.75 105.865002) (width 0.25) (layer F.Cu) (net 22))
 (segment (start 154.59 110.62) (end 161.995002 110.62) (width 0.25) (layer F.Cu) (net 22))
 (segment (start 154.5 94.75) (end 151.54 97.71) (width 0.25) (layer F.Cu) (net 32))
 (segment (start 151.54 97.71) (end 151.54 105.97) (width 0.25) (layer F.Cu) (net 32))
 (segment (start 154.5 90.5) (end 154.5 94.75) (width 0.25) (layer F.Cu) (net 32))
 (segment (start 148 101.570446) (end 146 101.570446) (width 0.25) (layer B.Cu) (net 35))
 (segment (start 148.25 103.75) (end 148.25 101.820446) (width 0.25) (layer B.Cu) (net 35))
 (segment (start 148.25 101.820446) (end 148 101.570446) (width 0.25) (layer B.Cu) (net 35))
 (segment (start 148.34 105.97) (end 148.34 103.84) (width 0.25) (layer F.Cu) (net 35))
 (segment (start 148.34 103.84) (end 148.25 103.75) (width 0.25) (layer F.Cu) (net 35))
 (via (at 148.25 103.75) (size 0.6) (drill 0.4) (layers F.Cu B.Cu) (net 35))
 (segment (start 149.94 105.97) (end 149.94 94.7864) (width 0.25) (layer F.Cu) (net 31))
 (segment (start 149.94 94.7864) (end 145.6536 90.5) (width 0.25) (layer F.Cu) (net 31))
 (segment (start 145.6536 90.5) (end 144.54 90.5) (width 0.25) (layer F.Cu) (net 31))
 (segment (start 142 90.5) (end 142 90.6524) (width 0.25) (layer F.Cu) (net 30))
 (segment (start 142 90.6524) (end 149.14 97.7924) (width 0.25) (layer F.Cu) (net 30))
 (segment (start 149.14 97.7924) (end 149.14 105.12) (width 0.25) (layer F.Cu) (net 30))
 (segment (start 149.14 105.12) (end 149.14 105.97) (width 0.25) (layer F.Cu) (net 30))
 (segment (start 157.5 130) (end 157.5 122) (width 1.5) (layer F.Cu) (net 2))
 (segment (start 158 103.7) (end 156.325 103.7) (width 0.25) (layer F.Cu) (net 2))
 (segment (start 156.325 103.7) (end 155 102.375) (width 0.25) (layer F.Cu) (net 2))
 (segment (start 155 102.375) (end 155 102.25) (width 0.25) (layer F.Cu) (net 2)))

